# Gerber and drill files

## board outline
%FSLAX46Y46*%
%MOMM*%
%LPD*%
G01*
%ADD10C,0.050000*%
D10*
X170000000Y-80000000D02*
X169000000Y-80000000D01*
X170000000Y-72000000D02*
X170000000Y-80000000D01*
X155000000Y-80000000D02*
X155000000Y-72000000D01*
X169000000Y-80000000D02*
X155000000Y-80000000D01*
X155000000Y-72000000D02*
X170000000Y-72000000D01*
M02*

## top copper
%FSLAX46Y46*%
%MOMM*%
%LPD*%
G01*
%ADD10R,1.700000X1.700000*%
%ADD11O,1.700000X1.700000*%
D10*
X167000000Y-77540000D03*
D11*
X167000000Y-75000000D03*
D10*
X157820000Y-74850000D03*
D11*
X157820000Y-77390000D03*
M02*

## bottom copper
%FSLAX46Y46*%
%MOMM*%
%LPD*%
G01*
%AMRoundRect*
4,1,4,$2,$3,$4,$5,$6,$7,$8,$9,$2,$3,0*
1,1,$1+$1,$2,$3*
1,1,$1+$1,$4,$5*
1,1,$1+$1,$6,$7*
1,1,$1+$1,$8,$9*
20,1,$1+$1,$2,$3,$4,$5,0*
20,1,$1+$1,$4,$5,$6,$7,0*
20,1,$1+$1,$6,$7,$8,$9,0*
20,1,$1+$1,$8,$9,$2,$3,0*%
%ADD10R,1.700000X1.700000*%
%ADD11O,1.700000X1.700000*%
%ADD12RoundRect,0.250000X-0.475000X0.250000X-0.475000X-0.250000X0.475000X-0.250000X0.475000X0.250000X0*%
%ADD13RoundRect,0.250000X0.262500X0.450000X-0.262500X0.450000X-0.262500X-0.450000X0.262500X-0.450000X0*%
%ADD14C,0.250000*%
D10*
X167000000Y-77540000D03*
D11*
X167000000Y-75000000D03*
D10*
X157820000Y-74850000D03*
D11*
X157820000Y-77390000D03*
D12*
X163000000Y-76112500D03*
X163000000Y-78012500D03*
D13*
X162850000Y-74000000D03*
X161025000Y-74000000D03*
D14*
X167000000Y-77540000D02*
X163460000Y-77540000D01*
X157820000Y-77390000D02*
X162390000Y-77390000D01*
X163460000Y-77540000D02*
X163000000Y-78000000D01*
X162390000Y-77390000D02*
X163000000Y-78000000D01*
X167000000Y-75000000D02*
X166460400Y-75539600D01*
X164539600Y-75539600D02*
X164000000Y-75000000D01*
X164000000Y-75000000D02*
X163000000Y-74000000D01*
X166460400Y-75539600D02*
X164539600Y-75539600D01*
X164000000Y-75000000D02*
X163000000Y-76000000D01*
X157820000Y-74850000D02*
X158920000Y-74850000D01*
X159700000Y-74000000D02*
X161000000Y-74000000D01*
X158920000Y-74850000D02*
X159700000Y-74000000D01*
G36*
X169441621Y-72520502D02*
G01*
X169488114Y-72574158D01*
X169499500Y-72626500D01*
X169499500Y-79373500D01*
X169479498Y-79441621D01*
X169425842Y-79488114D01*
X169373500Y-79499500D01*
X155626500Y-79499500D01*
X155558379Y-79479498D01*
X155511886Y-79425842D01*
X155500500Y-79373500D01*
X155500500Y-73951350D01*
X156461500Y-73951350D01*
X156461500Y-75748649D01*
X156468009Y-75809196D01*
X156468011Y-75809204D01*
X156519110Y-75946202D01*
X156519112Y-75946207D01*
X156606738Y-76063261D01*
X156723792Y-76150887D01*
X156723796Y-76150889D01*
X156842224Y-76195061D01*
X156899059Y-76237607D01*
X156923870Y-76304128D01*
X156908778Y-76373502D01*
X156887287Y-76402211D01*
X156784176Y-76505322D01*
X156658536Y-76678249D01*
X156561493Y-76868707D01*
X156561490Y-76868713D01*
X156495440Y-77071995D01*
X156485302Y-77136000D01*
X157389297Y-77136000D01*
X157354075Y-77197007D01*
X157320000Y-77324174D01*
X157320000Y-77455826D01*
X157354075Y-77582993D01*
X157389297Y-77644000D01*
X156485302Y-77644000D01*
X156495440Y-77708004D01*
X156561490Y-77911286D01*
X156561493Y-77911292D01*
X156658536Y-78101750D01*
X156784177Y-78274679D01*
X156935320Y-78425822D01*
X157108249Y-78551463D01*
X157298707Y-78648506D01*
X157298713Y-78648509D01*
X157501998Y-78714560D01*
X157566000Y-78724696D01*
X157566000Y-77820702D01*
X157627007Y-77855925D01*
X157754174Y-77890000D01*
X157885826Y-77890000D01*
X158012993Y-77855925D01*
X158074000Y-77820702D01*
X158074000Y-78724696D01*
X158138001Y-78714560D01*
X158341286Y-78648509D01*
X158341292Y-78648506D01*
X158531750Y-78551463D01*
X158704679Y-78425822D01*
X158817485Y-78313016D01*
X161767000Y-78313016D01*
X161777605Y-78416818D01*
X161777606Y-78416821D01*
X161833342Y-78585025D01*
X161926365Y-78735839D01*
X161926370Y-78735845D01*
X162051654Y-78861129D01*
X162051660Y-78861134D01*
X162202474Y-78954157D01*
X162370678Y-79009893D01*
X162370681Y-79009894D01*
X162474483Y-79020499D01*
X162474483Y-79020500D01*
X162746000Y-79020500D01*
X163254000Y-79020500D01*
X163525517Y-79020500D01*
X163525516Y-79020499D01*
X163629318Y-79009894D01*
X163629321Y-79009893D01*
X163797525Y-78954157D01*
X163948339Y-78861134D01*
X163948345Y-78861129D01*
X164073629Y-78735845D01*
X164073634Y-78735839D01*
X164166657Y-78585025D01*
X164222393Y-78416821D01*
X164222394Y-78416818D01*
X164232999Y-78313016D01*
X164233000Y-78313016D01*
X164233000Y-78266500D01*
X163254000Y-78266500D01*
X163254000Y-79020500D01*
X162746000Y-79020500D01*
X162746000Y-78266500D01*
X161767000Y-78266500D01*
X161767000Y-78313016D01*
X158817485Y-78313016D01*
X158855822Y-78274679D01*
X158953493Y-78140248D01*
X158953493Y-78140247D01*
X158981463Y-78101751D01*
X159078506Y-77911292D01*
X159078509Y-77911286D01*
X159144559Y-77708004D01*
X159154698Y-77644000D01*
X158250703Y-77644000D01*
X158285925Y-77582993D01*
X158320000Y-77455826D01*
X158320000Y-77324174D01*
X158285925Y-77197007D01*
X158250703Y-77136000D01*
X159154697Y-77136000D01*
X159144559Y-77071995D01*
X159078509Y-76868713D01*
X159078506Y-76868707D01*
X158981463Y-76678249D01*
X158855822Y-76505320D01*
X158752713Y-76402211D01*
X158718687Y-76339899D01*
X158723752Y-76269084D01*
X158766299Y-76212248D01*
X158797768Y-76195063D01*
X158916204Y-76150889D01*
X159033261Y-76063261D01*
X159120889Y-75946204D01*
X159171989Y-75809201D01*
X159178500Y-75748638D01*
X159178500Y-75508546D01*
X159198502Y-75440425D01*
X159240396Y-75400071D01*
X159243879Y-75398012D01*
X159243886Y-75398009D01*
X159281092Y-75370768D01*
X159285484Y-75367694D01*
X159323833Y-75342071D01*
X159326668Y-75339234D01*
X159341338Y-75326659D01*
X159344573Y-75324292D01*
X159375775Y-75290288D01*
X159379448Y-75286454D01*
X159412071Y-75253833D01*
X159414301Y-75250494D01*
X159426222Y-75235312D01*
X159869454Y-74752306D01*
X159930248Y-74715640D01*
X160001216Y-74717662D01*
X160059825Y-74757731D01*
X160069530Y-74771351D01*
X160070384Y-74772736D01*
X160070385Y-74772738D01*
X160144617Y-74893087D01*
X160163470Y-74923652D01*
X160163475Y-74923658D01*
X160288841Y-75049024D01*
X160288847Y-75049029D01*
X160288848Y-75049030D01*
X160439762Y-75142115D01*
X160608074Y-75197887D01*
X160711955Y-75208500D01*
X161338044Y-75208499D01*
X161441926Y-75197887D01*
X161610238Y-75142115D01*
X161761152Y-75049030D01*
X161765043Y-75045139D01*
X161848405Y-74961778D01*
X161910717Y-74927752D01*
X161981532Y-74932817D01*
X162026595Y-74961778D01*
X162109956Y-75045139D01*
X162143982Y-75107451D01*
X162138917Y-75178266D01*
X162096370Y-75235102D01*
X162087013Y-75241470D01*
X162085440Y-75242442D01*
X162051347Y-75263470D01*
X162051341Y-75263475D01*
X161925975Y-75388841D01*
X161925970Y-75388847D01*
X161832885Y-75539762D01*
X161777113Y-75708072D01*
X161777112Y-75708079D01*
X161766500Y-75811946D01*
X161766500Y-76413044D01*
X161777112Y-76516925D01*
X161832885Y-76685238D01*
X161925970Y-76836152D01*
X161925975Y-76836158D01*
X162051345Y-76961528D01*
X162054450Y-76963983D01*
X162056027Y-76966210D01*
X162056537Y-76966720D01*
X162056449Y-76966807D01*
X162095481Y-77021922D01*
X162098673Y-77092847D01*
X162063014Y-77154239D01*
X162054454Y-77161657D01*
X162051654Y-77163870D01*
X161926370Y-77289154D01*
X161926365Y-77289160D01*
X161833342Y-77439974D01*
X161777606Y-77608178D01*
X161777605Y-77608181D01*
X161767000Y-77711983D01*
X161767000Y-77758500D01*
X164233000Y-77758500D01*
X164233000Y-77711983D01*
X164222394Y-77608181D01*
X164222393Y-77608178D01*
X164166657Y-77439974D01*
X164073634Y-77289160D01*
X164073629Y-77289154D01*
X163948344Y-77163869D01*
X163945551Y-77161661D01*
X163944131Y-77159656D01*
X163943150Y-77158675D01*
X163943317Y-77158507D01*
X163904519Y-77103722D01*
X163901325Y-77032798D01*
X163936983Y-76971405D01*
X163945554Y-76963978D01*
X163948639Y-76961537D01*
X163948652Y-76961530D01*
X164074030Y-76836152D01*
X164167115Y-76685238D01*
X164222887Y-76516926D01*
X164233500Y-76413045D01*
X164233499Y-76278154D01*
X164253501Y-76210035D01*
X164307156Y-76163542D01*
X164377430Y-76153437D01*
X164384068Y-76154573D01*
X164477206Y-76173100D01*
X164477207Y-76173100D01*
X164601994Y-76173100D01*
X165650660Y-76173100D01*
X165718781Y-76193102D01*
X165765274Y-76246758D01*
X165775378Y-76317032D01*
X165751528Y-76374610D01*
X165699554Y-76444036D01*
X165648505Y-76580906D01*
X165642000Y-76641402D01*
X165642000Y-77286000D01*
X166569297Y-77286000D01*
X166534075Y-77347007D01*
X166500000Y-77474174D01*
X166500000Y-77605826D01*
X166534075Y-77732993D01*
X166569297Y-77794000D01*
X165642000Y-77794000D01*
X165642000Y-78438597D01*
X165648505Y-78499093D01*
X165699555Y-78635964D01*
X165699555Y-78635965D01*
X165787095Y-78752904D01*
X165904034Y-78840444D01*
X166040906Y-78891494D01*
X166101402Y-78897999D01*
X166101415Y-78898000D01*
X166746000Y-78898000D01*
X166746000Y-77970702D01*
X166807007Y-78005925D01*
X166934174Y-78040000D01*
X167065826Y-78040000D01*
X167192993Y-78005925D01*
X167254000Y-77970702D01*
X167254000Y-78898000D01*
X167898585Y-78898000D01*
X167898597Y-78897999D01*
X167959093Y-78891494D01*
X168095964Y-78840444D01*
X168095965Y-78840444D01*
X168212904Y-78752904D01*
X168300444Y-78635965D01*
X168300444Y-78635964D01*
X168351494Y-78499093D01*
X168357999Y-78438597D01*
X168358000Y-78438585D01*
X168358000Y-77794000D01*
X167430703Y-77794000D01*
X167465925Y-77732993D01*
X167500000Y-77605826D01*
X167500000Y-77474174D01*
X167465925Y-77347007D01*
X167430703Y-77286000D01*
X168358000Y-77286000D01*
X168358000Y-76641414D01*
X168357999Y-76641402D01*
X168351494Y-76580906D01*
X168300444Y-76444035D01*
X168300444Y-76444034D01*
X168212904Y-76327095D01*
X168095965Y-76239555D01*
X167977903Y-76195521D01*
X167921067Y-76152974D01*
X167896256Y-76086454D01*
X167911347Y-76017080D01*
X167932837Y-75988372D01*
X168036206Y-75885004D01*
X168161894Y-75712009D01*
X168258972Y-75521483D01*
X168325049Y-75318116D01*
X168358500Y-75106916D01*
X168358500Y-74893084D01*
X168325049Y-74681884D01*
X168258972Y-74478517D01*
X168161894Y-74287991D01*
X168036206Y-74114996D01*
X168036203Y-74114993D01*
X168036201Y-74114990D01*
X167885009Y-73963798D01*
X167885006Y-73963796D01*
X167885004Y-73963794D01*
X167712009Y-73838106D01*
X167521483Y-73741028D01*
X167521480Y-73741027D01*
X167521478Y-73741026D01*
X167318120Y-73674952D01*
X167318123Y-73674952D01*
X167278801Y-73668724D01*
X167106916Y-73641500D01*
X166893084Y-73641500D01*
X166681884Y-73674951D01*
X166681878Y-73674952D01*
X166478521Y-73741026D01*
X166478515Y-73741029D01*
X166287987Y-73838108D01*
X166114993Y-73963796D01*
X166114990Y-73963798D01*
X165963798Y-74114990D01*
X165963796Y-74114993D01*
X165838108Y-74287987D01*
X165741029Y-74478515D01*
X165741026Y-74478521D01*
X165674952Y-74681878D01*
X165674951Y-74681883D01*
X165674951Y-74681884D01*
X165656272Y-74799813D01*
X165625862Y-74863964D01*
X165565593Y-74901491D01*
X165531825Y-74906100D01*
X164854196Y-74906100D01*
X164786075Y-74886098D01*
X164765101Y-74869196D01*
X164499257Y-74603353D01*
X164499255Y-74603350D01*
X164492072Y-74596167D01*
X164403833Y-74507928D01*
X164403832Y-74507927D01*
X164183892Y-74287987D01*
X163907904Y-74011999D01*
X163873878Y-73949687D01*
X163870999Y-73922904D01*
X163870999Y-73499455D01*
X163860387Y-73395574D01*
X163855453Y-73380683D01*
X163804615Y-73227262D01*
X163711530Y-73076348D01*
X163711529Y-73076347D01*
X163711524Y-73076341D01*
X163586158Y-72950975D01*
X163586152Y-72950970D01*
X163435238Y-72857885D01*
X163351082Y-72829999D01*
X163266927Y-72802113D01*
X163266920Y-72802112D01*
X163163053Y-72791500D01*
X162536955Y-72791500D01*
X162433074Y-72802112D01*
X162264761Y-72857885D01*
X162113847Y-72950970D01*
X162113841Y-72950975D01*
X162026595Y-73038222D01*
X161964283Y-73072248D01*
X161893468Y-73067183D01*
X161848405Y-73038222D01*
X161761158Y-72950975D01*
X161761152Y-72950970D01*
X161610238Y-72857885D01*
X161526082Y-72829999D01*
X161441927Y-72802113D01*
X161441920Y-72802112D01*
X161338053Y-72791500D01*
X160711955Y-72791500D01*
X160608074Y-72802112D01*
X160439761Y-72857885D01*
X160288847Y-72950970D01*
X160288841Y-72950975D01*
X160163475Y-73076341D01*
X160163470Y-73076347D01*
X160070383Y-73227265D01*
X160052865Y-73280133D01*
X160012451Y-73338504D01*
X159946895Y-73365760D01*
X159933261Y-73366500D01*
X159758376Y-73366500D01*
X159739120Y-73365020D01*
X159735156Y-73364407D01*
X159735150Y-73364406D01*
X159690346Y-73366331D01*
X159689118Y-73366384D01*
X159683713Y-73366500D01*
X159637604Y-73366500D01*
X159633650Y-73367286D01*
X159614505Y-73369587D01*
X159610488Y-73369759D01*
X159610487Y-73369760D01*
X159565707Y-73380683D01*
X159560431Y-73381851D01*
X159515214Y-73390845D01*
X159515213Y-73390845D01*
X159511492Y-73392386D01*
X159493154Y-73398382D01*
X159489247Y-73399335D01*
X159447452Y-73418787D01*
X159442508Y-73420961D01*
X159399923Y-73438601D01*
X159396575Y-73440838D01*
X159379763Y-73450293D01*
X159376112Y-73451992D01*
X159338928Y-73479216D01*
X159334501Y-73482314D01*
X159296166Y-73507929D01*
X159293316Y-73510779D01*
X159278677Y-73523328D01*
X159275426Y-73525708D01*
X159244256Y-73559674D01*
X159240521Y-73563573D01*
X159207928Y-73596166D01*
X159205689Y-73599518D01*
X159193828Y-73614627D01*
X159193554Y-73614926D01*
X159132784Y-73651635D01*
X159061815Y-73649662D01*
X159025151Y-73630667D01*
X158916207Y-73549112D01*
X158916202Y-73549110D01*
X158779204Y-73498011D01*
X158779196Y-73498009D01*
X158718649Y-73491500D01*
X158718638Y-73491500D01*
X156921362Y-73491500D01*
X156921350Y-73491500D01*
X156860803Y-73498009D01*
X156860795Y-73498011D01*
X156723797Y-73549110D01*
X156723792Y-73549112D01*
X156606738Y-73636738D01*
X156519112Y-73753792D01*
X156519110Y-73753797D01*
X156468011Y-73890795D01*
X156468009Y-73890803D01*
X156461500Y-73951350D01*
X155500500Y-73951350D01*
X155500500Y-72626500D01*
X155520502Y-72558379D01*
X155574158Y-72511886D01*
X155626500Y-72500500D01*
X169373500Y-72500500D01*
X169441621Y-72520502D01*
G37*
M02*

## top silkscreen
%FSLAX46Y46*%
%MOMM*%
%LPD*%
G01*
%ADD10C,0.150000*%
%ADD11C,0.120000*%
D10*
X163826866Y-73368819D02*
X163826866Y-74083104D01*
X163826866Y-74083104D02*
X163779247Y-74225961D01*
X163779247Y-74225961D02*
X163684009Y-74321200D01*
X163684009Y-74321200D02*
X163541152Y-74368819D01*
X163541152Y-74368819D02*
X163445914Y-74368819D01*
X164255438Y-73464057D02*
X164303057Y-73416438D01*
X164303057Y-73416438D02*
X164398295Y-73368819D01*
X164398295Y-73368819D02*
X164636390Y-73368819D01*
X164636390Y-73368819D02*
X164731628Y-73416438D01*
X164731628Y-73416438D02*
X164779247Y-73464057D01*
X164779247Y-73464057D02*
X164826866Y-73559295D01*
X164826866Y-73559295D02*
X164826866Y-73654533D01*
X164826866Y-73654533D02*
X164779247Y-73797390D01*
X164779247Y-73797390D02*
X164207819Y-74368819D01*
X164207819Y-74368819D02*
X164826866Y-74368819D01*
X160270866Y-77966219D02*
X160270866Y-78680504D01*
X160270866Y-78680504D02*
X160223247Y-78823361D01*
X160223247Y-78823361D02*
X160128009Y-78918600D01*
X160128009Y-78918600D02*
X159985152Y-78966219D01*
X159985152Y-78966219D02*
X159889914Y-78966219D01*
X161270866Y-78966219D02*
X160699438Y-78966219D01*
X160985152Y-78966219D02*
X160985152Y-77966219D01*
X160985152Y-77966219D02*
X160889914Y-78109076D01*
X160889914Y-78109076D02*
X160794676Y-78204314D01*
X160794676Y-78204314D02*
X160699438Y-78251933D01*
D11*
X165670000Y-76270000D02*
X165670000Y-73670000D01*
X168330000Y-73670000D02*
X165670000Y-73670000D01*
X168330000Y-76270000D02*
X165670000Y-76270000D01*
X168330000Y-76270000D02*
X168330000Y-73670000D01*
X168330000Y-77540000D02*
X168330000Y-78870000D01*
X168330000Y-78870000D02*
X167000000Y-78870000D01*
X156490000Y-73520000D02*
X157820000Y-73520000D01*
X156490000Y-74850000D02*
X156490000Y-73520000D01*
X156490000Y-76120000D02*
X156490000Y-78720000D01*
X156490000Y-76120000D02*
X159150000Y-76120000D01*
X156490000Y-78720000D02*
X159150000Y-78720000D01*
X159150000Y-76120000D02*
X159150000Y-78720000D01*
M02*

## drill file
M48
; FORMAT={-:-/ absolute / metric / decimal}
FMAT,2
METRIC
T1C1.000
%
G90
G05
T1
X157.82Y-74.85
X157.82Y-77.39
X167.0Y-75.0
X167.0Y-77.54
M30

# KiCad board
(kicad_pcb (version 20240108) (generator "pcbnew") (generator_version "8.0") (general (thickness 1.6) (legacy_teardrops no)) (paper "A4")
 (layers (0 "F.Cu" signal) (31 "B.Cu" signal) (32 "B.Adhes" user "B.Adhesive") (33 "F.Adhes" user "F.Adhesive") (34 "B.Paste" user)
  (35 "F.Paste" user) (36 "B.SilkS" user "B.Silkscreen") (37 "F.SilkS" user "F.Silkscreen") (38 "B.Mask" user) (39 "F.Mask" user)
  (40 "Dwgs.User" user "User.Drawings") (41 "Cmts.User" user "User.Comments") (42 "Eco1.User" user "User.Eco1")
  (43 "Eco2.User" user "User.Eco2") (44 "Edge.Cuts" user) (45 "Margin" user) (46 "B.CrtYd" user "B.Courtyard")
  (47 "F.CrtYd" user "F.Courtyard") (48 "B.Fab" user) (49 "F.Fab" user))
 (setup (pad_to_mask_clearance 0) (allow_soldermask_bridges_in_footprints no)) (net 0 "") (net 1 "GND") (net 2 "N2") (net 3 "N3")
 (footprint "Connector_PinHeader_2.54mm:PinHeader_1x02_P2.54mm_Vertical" (layer "F.Cu") (at 167 77.54 180)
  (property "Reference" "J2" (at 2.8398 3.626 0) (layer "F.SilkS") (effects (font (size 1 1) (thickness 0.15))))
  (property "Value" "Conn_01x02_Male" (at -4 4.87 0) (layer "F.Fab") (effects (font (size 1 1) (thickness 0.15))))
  (fp_line (start 1.33 1.27) (end 1.33 3.87) (stroke (width 0.12) (type solid)) (layer "F.SilkS"))
  (fp_line (start -1.33 3.87) (end 1.33 3.87) (stroke (width 0.12) (type solid)) (layer "F.SilkS"))
  (fp_line (start -1.33 1.27) (end 1.33 1.27) (stroke (width 0.12) (type solid)) (layer "F.SilkS"))
  (fp_line (start -1.33 1.27) (end -1.33 3.87) (stroke (width 0.12) (type solid)) (layer "F.SilkS"))
  (fp_line (start -1.33 0) (end -1.33 -1.33) (stroke (width 0.12) (type solid)) (layer "F.SilkS"))
  (fp_line (start -1.33 -1.33) (end 0 -1.33) (stroke (width 0.12) (type solid)) (layer "F.SilkS"))
  (pad "1" thru_hole rect (at 0 0 180) (size 1.7 1.7) (drill 1) (layers "*.Cu" "*.Mask") (remove_unused_layers no) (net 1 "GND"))
  (pad "2" thru_hole oval (at 0 2.54 180) (size 1.7 1.7) (drill 1) (layers "*.Cu" "*.Mask") (remove_unused_layers no) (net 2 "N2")))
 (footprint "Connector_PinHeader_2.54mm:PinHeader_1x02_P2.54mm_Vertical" (layer "F.Cu") (at 157.82 74.85)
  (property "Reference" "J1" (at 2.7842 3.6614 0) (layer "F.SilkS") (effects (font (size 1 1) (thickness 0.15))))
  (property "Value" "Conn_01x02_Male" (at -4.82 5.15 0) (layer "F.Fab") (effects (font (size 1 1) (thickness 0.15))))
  (fp_line (start -1.33 -1.33) (end 0 -1.33) (stroke (width 0.12) (type solid)) (layer "F.SilkS"))
  (fp_line (start -1.33 0) (end -1.33 -1.33) (stroke (width 0.12) (type solid)) (layer "F.SilkS"))
  (fp_line (start -1.33 1.27) (end -1.33 3.87) (stroke (width 0.12) (type solid)) (layer "F.SilkS"))
  (fp_line (start -1.33 1.27) (end 1.33 1.27) (stroke (width 0.12) (type solid)) (layer "F.SilkS"))
  (fp_line (start -1.33 3.87) (end 1.33 3.87) (stroke (width 0.12) (type solid)) (layer "F.SilkS"))
  (fp_line (start 1.33 1.27) (end 1.33 3.87) (stroke (width 0.12) (type solid)) (layer "F.SilkS"))
  (pad "1" thru_hole rect (at 0 0) (size 1.7 1.7) (drill 1) (layers "*.Cu" "*.Mask") (remove_unused_layers no) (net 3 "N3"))
  (pad "2" thru_hole oval (at 0 2.54) (size 1.7 1.7) (drill 1) (layers "*.Cu" "*.Mask") (remove_unused_layers no) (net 1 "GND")))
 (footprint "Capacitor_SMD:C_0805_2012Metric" (layer "B.Cu") (at 163 77.0625 -90)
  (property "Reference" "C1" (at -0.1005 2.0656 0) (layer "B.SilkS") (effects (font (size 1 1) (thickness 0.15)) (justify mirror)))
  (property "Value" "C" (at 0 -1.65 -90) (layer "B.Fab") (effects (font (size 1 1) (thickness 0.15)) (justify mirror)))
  (pad "1" smd roundrect (at -0.95 0 270) (size 1 1.45) (layers "B.Cu" "B.Paste" "B.Mask") (roundrect_rratio 0.25) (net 2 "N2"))
  (pad "2" smd roundrect (at 0.95 0 270) (size 1 1.45) (layers "B.Cu" "B.Paste" "B.Mask") (roundrect_rratio 0.25) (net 1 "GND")))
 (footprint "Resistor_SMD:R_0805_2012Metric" (layer "B.Cu") (at 161.9375 74 180)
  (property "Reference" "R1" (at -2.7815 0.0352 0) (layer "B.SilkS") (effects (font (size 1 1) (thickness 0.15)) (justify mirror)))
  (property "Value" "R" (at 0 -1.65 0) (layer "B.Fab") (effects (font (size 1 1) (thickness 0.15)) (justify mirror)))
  (pad "1" smd roundrect (at -0.9125 0 180) (size 1.025 1.4) (layers "B.Cu" "B.Paste" "B.Mask") (roundrect_rratio 0.243902) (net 2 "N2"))
  (pad "2" smd roundrect (at 0.9125 0 180) (size 1.025 1.4) (layers "B.Cu" "B.Paste" "B.Mask") (roundrect_rratio 0.243902) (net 3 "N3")))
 (gr_line (start 170 80) (end 169 80) (stroke (width 0.05) (type solid)) (layer "Edge.Cuts"))
 (gr_line (start 170 72) (end 170 80) (stroke (width 0.05) (type solid)) (layer "Edge.Cuts"))
 (gr_line (start 155 80) (end 155 72) (stroke (width 0.05) (type solid)) (layer "Edge.Cuts"))
 (gr_line (start 169 80) (end 155 80) (stroke (width 0.05) (type solid)) (layer "Edge.Cuts"))
 (gr_line (start 155 72) (end 170 72) (stroke (width 0.05) (type solid)) (layer "Edge.Cuts"))
 (segment (start 167 77.54) (end 163.46 77.54) (width 0.25) (layer "B.Cu") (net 1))
 (segment (start 157.82 77.39) (end 162.39 77.39) (width 0.25) (layer "B.Cu") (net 1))
 (segment (start 163.46 77.54) (end 163 78) (width 0.25) (layer "B.Cu") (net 1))
 (segment (start 162.39 77.39) (end 163 78) (width 0.25) (layer "B.Cu") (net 1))
 (segment (start 167 75) (end 166.4604 75.5396) (width 0.25) (layer "B.Cu") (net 2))
 (segment (start 164.5396 75.5396) (end 164 75) (width 0.25) (layer "B.Cu") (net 2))
 (segment (start 164 75) (end 163 74) (width 0.25) (layer "B.Cu") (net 2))
 (segment (start 166.4604 75.5396) (end 164.5396 75.5396) (width 0.25) (layer "B.Cu") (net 2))
 (segment (start 164 75) (end 163 76) (width 0.25) (layer "B.Cu") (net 2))
 (segment (start 157.82 74.85) (end 158.92 74.85) (width 0.25) (layer "B.Cu") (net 3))
 (segment (start 159.7 74) (end 161 74) (width 0.25) (layer "B.Cu") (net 3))
 (segment (start 158.92 74.85) (end 159.7 74) (width 0.25) (layer "B.Cu") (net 3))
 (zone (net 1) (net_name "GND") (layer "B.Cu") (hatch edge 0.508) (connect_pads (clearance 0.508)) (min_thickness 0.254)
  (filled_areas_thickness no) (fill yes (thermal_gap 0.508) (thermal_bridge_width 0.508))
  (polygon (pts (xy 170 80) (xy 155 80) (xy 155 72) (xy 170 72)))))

